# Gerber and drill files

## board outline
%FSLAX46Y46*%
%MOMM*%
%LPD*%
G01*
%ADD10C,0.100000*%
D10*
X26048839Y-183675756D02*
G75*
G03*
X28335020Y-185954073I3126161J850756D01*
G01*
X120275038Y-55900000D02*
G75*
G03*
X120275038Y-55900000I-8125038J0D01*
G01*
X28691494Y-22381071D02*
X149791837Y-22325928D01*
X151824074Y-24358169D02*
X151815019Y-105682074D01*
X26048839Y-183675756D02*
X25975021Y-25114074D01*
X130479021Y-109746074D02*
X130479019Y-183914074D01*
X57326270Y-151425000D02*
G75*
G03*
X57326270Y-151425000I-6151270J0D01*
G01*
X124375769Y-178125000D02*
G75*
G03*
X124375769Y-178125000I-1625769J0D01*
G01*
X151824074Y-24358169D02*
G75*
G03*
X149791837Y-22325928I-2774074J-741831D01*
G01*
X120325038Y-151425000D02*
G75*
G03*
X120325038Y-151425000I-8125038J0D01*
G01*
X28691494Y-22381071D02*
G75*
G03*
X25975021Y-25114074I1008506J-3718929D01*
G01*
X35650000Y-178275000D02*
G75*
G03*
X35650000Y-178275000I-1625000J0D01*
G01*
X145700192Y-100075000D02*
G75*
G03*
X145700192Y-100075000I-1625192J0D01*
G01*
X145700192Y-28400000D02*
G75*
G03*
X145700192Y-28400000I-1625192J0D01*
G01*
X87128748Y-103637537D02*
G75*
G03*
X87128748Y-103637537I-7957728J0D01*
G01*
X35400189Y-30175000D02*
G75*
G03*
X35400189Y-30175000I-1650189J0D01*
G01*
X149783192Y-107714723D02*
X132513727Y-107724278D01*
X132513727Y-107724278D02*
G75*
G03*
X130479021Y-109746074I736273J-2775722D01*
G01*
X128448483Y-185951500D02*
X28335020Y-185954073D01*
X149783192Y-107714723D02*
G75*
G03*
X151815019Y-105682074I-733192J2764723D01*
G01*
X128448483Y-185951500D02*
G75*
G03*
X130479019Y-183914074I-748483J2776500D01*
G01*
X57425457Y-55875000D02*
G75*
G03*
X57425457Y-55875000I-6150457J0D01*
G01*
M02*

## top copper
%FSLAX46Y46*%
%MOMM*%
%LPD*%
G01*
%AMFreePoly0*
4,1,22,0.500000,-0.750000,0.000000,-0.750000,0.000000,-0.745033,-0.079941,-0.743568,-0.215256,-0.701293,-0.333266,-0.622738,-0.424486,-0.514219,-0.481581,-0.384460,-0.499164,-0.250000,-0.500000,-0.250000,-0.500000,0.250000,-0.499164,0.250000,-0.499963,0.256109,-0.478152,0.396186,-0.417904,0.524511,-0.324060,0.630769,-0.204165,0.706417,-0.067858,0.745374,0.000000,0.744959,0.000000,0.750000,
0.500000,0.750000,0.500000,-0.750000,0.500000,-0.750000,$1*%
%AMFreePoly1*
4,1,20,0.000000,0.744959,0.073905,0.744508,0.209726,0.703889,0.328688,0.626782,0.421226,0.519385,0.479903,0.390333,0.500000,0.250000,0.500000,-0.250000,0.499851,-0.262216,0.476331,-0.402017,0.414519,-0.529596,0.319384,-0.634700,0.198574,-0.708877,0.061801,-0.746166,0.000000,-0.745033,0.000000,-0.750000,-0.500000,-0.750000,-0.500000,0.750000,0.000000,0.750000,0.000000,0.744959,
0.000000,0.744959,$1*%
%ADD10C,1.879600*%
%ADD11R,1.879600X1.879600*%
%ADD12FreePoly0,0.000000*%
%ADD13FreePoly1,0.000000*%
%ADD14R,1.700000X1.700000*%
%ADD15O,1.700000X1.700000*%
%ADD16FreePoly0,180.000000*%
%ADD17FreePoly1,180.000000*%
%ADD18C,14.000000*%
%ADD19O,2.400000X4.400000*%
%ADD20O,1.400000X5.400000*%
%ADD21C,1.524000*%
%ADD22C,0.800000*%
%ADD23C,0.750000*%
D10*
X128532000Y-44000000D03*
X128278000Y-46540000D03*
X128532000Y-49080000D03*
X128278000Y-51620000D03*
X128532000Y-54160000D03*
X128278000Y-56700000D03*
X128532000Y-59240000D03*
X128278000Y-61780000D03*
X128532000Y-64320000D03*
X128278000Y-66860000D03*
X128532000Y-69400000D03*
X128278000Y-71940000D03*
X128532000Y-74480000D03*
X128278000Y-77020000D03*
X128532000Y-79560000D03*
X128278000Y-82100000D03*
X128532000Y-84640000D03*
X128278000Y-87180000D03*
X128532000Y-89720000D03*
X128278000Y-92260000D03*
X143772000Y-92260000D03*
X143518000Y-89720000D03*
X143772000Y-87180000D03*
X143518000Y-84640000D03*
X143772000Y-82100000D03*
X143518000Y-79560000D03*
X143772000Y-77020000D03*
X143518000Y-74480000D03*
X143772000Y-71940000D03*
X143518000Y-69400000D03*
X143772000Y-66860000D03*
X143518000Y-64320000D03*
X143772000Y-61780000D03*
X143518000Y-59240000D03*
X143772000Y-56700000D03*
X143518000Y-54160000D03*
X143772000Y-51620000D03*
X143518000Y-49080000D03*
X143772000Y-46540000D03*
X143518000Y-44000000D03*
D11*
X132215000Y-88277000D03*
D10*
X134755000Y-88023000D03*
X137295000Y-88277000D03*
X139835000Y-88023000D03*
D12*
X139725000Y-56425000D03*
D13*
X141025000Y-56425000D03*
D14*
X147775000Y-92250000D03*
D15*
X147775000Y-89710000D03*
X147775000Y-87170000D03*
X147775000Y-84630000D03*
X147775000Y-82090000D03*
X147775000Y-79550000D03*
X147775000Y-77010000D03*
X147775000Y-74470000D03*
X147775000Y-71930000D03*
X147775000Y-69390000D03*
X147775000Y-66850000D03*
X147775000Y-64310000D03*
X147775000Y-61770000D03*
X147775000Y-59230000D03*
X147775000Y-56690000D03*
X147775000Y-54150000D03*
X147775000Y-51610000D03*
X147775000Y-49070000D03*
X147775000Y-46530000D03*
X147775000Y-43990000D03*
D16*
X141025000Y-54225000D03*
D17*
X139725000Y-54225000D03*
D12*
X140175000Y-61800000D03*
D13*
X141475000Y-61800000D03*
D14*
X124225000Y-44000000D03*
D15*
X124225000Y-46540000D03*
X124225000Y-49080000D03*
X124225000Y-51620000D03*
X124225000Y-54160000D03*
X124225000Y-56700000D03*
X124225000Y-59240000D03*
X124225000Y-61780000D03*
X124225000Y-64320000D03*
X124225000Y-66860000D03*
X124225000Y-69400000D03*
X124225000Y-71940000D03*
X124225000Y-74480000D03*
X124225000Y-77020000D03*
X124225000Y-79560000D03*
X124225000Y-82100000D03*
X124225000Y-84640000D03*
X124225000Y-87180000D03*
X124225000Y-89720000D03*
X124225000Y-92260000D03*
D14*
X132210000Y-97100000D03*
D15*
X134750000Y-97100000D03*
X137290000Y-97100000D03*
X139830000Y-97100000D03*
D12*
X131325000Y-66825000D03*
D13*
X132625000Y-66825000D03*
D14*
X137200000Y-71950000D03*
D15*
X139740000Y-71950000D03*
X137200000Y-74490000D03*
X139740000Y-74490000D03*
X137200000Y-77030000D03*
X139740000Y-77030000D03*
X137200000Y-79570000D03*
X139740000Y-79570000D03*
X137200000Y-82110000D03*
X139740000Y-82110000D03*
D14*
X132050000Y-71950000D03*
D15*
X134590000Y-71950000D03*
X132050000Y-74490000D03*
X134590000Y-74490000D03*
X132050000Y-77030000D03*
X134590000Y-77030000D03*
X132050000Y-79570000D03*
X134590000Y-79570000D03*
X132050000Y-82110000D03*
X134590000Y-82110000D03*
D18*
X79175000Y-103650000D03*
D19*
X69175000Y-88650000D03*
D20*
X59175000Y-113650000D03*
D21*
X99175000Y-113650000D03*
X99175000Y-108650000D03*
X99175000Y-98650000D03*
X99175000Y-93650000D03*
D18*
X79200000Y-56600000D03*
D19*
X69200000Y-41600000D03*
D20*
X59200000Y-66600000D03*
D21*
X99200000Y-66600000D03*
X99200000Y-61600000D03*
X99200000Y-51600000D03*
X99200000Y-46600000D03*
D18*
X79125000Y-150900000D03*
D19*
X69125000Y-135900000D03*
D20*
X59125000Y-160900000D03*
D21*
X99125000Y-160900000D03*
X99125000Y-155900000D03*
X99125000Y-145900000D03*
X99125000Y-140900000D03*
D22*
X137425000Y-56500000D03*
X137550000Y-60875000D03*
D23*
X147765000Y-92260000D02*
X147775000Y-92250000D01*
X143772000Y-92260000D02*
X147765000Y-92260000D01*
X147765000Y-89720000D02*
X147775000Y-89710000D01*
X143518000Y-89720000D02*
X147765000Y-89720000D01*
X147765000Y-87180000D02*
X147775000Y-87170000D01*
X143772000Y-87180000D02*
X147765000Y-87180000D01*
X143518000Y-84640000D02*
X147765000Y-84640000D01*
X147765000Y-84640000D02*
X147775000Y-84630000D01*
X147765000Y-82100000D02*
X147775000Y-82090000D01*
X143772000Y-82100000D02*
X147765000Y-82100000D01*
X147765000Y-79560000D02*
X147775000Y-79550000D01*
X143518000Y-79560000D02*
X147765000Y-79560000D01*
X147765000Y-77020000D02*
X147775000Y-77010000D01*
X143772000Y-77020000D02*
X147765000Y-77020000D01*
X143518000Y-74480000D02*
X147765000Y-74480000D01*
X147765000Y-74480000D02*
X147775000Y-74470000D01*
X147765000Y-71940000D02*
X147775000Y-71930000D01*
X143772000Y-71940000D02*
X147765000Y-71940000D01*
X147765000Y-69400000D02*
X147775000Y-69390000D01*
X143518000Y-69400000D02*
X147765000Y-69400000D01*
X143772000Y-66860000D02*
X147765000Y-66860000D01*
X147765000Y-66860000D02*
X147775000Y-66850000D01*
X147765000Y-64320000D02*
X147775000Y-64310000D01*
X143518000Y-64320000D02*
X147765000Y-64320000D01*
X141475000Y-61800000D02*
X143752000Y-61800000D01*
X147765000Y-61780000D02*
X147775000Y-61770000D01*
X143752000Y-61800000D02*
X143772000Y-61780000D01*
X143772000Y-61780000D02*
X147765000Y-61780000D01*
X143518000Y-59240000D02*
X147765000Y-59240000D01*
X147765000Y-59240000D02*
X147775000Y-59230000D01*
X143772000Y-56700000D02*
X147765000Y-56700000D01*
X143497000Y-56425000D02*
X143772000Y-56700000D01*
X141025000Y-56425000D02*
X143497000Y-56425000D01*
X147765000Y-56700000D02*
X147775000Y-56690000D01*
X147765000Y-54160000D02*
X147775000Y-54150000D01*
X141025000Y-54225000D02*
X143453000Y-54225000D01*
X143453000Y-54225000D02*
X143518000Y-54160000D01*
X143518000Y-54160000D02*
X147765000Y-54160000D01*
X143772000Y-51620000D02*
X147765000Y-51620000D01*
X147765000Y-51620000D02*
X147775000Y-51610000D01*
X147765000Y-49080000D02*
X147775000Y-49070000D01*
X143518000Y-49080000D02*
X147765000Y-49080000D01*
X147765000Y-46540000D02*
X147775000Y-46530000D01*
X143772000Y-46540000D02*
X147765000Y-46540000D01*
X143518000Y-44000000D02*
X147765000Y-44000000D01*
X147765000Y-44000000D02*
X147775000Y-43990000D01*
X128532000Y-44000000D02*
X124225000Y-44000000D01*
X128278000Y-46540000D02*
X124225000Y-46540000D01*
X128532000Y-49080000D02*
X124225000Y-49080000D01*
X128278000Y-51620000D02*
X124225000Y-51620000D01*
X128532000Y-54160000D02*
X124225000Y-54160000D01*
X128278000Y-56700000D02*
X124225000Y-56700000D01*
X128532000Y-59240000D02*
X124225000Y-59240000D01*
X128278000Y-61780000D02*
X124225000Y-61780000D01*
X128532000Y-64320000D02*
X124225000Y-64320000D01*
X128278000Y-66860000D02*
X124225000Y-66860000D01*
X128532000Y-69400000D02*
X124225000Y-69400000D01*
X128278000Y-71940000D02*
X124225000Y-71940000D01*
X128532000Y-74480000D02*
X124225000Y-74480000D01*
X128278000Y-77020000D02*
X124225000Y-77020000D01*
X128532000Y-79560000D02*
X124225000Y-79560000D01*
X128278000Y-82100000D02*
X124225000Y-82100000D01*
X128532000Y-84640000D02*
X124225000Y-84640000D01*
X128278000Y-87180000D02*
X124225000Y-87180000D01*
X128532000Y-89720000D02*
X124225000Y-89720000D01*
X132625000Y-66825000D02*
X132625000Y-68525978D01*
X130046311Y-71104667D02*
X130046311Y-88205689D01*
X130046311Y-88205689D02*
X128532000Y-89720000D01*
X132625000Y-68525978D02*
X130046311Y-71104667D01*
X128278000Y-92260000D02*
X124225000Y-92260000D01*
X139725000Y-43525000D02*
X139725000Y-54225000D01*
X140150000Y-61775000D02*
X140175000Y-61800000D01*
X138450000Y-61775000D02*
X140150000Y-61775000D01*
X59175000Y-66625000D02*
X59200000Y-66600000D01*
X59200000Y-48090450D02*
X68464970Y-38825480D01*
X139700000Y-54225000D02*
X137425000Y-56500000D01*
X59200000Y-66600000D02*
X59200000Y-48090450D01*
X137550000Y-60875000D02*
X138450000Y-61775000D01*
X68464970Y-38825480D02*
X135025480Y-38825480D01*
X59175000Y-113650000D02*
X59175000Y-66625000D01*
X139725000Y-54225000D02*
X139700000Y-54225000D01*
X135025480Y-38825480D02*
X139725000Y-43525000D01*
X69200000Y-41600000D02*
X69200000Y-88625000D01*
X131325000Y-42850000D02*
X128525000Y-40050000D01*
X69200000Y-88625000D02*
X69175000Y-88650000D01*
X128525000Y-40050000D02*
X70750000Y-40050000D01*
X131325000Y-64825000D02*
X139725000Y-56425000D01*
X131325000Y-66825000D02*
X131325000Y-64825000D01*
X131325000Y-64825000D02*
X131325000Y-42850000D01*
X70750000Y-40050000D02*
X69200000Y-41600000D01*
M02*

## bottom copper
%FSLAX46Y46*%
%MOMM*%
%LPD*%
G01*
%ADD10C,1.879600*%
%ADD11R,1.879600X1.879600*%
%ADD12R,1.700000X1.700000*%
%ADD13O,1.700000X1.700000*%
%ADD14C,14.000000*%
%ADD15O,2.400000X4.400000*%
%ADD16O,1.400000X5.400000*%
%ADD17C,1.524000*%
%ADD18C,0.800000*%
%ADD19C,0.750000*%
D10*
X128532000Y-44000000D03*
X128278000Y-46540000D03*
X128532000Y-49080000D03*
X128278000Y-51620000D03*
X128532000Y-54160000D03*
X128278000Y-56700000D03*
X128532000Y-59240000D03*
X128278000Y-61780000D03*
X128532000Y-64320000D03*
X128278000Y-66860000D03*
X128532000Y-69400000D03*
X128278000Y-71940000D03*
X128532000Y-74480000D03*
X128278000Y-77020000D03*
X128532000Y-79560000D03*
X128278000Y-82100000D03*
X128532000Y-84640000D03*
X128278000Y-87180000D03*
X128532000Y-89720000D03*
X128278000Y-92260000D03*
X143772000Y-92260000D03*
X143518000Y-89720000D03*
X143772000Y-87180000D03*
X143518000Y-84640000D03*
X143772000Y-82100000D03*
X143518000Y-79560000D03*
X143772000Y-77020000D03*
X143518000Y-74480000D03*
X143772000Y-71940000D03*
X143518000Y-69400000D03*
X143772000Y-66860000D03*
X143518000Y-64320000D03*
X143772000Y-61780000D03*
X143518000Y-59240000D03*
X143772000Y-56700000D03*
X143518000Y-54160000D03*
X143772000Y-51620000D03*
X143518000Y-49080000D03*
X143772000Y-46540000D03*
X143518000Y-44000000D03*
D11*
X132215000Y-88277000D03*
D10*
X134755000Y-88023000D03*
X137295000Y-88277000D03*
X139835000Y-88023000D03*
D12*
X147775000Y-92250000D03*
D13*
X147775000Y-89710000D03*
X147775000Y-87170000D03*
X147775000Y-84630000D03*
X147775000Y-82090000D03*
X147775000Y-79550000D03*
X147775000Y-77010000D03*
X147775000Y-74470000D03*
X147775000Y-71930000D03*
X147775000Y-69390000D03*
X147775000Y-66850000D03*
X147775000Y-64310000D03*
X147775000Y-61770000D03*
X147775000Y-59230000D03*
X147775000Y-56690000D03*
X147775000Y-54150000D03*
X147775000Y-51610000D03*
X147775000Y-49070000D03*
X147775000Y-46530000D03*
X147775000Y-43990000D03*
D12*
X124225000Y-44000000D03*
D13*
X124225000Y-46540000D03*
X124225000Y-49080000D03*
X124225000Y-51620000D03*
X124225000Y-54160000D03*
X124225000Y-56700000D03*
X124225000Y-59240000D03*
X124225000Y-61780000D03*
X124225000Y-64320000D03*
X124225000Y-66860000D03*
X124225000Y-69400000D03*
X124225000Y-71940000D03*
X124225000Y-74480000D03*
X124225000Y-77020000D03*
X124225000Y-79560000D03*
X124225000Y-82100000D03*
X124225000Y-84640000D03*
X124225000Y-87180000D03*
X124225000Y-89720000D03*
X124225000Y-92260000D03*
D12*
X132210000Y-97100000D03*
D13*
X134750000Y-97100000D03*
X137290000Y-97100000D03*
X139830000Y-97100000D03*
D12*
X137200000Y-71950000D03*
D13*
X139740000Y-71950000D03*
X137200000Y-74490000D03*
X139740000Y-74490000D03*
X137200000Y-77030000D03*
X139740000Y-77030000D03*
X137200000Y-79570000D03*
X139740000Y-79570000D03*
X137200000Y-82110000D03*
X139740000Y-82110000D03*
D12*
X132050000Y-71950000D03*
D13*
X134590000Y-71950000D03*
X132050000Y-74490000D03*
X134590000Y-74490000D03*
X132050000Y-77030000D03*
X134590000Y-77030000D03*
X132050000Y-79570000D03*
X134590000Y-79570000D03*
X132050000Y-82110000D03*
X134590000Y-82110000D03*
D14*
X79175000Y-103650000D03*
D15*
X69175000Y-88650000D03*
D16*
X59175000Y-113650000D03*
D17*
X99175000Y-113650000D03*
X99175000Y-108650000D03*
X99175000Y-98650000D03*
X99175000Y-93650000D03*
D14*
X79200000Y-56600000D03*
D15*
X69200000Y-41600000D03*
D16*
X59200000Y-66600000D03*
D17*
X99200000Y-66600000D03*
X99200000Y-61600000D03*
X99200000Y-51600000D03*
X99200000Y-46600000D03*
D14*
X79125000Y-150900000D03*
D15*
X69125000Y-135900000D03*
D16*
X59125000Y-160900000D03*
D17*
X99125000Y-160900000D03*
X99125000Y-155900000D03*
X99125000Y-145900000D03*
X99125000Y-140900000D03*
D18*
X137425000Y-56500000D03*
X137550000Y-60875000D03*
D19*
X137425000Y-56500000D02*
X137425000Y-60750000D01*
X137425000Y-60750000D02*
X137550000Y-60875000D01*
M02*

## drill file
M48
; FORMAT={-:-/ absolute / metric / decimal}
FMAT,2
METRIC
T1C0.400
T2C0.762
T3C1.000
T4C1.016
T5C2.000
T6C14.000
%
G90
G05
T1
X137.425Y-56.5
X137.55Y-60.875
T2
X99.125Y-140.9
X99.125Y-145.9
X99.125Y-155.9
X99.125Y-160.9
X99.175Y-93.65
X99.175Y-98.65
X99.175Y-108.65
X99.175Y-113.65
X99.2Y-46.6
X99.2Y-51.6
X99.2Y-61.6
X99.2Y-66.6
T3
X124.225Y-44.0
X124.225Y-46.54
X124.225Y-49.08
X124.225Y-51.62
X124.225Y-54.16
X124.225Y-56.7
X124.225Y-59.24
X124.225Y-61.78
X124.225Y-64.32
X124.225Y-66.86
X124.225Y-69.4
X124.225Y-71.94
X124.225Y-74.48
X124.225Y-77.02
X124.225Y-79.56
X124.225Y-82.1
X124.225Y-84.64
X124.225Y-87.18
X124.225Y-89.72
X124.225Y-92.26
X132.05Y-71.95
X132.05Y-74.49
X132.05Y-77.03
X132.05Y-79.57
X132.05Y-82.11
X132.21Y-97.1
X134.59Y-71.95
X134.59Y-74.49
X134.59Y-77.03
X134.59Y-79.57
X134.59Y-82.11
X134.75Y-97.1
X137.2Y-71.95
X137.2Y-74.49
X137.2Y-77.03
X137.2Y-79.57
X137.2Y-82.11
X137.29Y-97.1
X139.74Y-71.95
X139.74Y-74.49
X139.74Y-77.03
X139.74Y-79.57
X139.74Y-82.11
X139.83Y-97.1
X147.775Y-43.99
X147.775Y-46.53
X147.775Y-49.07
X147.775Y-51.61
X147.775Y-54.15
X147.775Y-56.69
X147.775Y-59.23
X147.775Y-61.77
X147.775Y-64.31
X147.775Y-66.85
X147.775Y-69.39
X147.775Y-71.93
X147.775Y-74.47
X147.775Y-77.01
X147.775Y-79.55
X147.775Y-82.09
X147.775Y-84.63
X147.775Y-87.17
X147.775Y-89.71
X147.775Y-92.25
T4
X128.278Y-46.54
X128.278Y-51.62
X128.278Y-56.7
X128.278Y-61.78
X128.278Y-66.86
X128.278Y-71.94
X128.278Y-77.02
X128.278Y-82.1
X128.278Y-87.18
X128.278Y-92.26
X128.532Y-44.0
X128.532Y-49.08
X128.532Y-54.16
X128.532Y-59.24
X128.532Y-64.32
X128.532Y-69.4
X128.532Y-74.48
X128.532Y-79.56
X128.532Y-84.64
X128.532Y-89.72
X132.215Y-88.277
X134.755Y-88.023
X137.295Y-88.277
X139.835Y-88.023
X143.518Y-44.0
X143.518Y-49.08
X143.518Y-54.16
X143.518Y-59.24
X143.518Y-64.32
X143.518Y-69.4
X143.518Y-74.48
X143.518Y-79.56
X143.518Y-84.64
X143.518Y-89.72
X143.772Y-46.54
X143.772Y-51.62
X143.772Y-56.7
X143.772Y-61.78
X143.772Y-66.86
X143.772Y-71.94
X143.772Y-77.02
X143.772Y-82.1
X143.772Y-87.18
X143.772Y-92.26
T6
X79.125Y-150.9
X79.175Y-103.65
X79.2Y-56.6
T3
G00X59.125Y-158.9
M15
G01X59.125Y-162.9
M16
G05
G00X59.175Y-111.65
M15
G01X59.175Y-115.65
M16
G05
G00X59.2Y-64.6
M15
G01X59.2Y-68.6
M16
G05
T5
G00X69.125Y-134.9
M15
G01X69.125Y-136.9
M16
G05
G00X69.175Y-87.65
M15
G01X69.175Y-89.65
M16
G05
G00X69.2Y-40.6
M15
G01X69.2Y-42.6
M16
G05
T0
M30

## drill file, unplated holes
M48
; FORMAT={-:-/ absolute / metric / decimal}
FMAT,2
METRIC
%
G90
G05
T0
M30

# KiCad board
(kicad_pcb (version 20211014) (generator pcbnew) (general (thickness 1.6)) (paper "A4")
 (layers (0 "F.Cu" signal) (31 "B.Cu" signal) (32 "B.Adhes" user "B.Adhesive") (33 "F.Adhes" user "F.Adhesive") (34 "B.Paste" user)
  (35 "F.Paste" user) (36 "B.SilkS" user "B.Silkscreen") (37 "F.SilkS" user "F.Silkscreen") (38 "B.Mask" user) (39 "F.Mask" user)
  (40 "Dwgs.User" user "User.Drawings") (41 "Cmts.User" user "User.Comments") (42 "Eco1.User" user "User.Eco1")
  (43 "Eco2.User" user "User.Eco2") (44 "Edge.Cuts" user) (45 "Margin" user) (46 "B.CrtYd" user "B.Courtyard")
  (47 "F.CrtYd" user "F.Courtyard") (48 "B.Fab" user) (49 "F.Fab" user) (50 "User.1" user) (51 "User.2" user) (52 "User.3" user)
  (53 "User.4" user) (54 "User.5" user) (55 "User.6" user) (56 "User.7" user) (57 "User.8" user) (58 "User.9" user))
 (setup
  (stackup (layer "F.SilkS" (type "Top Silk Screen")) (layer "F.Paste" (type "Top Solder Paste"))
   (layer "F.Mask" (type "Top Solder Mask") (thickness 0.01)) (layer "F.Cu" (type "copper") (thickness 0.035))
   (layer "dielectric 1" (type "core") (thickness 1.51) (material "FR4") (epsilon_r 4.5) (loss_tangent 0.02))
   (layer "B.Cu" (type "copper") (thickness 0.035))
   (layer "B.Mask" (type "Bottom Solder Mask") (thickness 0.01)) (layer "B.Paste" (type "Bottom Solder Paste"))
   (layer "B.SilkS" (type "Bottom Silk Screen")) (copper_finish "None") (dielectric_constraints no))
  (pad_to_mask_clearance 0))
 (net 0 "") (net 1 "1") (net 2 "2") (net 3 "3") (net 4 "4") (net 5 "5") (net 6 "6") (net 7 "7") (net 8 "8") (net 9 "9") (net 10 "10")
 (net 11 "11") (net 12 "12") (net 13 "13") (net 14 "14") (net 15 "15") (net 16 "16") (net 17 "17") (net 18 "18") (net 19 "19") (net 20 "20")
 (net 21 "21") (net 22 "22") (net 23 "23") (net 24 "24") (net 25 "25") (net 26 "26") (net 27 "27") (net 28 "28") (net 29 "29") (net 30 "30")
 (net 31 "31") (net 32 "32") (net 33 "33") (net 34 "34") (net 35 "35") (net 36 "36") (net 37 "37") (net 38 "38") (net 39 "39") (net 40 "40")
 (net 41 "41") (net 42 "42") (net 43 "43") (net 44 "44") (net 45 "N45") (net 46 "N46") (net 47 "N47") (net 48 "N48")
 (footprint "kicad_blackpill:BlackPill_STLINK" (layer "F.Cu") (at 136.025 69.1)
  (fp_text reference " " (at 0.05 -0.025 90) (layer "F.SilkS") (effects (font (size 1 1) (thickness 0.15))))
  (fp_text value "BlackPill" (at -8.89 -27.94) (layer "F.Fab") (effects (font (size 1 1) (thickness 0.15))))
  (pad "1" thru_hole circle (at -7.493 -25.1 270) (size 1.8796 1.8796) (drill 1.016) (layers *.Cu *.Mask) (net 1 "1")
   (solder_mask_margin 0.1016))
  (pad "2" thru_hole circle (at -7.747 -22.56 270) (size 1.8796 1.8796) (drill 1.016) (layers *.Cu *.Mask) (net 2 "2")
   (solder_mask_margin 0.1016))
  (pad "3" thru_hole circle (at -7.493 -20.02 270) (size 1.8796 1.8796) (drill 1.016) (layers *.Cu *.Mask) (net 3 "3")
   (solder_mask_margin 0.1016))
  (pad "4" thru_hole circle (at -7.747 -17.48 270) (size 1.8796 1.8796) (drill 1.016) (layers *.Cu *.Mask) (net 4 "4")
   (solder_mask_margin 0.1016))
  (pad "5" thru_hole circle (at -7.493 -14.94 270) (size 1.8796 1.8796) (drill 1.016) (layers *.Cu *.Mask) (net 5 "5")
   (solder_mask_margin 0.1016))
  (pad "6" thru_hole circle (at -7.747 -12.4 270) (size 1.8796 1.8796) (drill 1.016) (layers *.Cu *.Mask) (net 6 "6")
   (solder_mask_margin 0.1016))
  (pad "7" thru_hole circle (at -7.493 -9.86 270) (size 1.8796 1.8796) (drill 1.016) (layers *.Cu *.Mask) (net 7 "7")
   (solder_mask_margin 0.1016))
  (pad "8" thru_hole circle (at -7.747 -7.32 270) (size 1.8796 1.8796) (drill 1.016) (layers *.Cu *.Mask) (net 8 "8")
   (solder_mask_margin 0.1016))
  (pad "9" thru_hole circle (at -7.493 -4.78 270) (size 1.8796 1.8796) (drill 1.016) (layers *.Cu *.Mask) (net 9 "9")
   (solder_mask_margin 0.1016))
  (pad "10" thru_hole circle (at -7.747 -2.24 270) (size 1.8796 1.8796) (drill 1.016) (layers *.Cu *.Mask) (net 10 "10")
   (solder_mask_margin 0.1016))
  (pad "11" thru_hole circle (at -7.493 0.3 270) (size 1.8796 1.8796) (drill 1.016) (layers *.Cu *.Mask) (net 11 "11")
   (solder_mask_margin 0.1016))
  (pad "12" thru_hole circle (at -7.747 2.84 270) (size 1.8796 1.8796) (drill 1.016) (layers *.Cu *.Mask) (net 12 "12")
   (solder_mask_margin 0.1016))
  (pad "13" thru_hole circle (at -7.493 5.38 270) (size 1.8796 1.8796) (drill 1.016) (layers *.Cu *.Mask) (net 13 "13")
   (solder_mask_margin 0.1016))
  (pad "14" thru_hole circle (at -7.747 7.92 270) (size 1.8796 1.8796) (drill 1.016) (layers *.Cu *.Mask) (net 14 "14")
   (solder_mask_margin 0.1016))
  (pad "15" thru_hole circle (at -7.493 10.46 270) (size 1.8796 1.8796) (drill 1.016) (layers *.Cu *.Mask) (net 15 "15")
   (solder_mask_margin 0.1016))
  (pad "16" thru_hole circle (at -7.747 13 270) (size 1.8796 1.8796) (drill 1.016) (layers *.Cu *.Mask) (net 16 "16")
   (solder_mask_margin 0.1016))
  (pad "17" thru_hole circle (at -7.493 15.54 270) (size 1.8796 1.8796) (drill 1.016) (layers *.Cu *.Mask) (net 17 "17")
   (solder_mask_margin 0.1016))
  (pad "18" thru_hole circle (at -7.747 18.08 270) (size 1.8796 1.8796) (drill 1.016) (layers *.Cu *.Mask) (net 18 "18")
   (solder_mask_margin 0.1016))
  (pad "19" thru_hole circle (at -7.493 20.62 270) (size 1.8796 1.8796) (drill 1.016) (layers *.Cu *.Mask) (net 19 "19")
   (solder_mask_margin 0.1016))
  (pad "20" thru_hole circle (at -7.747 23.16 270) (size 1.8796 1.8796) (drill 1.016) (layers *.Cu *.Mask) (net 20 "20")
   (solder_mask_margin 0.1016))
  (pad "21" thru_hole circle (at 7.747 23.16 90) (size 1.8796 1.8796) (drill 1.016) (layers *.Cu *.Mask) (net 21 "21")
   (solder_mask_margin 0.1016))
  (pad "22" thru_hole circle (at 7.493 20.62 90) (size 1.8796 1.8796) (drill 1.016) (layers *.Cu *.Mask) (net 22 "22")
   (solder_mask_margin 0.1016))
  (pad "23" thru_hole circle (at 7.747 18.08 90) (size 1.8796 1.8796) (drill 1.016) (layers *.Cu *.Mask) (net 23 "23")
   (solder_mask_margin 0.1016))
  (pad "24" thru_hole circle (at 7.493 15.54 90) (size 1.8796 1.8796) (drill 1.016) (layers *.Cu *.Mask) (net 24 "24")
   (solder_mask_margin 0.1016))
  (pad "25" thru_hole circle (at 7.747 13 90) (size 1.8796 1.8796) (drill 1.016) (layers *.Cu *.Mask) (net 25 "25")
   (solder_mask_margin 0.1016))
  (pad "26" thru_hole circle (at 7.493 10.46 90) (size 1.8796 1.8796) (drill 1.016) (layers *.Cu *.Mask) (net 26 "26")
   (solder_mask_margin 0.1016))
  (pad "27" thru_hole circle (at 7.747 7.92 90) (size 1.8796 1.8796) (drill 1.016) (layers *.Cu *.Mask) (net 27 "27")
   (solder_mask_margin 0.1016))
  (pad "28" thru_hole circle (at 7.493 5.38 90) (size 1.8796 1.8796) (drill 1.016) (layers *.Cu *.Mask) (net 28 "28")
   (solder_mask_margin 0.1016))
  (pad "29" thru_hole circle (at 7.747 2.84 90) (size 1.8796 1.8796) (drill 1.016) (layers *.Cu *.Mask) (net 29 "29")
   (solder_mask_margin 0.1016))
  (pad "30" thru_hole circle (at 7.493 0.3 90) (size 1.8796 1.8796) (drill 1.016) (layers *.Cu *.Mask) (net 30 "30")
   (solder_mask_margin 0.1016))
  (pad "31" thru_hole circle (at 7.747 -2.24 90) (size 1.8796 1.8796) (drill 1.016) (layers *.Cu *.Mask) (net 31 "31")
   (solder_mask_margin 0.1016))
  (pad "32" thru_hole circle (at 7.493 -4.78 90) (size 1.8796 1.8796) (drill 1.016) (layers *.Cu *.Mask) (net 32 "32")
   (solder_mask_margin 0.1016))
  (pad "33" thru_hole circle (at 7.747 -7.32 90) (size 1.8796 1.8796) (drill 1.016) (layers *.Cu *.Mask) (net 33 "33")
   (solder_mask_margin 0.1016))
  (pad "34" thru_hole circle (at 7.493 -9.86 90) (size 1.8796 1.8796) (drill 1.016) (layers *.Cu *.Mask) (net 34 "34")
   (solder_mask_margin 0.1016))
  (pad "35" thru_hole circle (at 7.747 -12.4 90) (size 1.8796 1.8796) (drill 1.016) (layers *.Cu *.Mask) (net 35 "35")
   (solder_mask_margin 0.1016))
  (pad "36" thru_hole circle (at 7.493 -14.94 90) (size 1.8796 1.8796) (drill 1.016) (layers *.Cu *.Mask) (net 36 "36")
   (solder_mask_margin 0.1016))
  (pad "37" thru_hole circle (at 7.747 -17.48 90) (size 1.8796 1.8796) (drill 1.016) (layers *.Cu *.Mask) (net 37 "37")
   (solder_mask_margin 0.1016))
  (pad "38" thru_hole circle (at 7.493 -20.02 90) (size 1.8796 1.8796) (drill 1.016) (layers *.Cu *.Mask) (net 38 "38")
   (solder_mask_margin 0.1016))
  (pad "39" thru_hole circle (at 7.747 -22.56 90) (size 1.8796 1.8796) (drill 1.016) (layers *.Cu *.Mask) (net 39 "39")
   (solder_mask_margin 0.1016))
  (pad "40" thru_hole circle (at 7.493 -25.1 90) (size 1.8796 1.8796) (drill 1.016) (layers *.Cu *.Mask) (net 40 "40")
   (solder_mask_margin 0.1016))
  (pad "41" thru_hole rect (at -3.81 19.177 90) (size 1.8796 1.8796) (drill 1.016) (layers *.Cu *.Mask) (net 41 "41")
   (solder_mask_margin 0.1016))
  (pad "42" thru_hole circle (at -1.27 18.923 90) (size 1.8796 1.8796) (drill 1.016) (layers *.Cu *.Mask) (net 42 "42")
   (solder_mask_margin 0.1016))
  (pad "43" thru_hole circle (at 1.27 19.177 90) (size 1.8796 1.8796) (drill 1.016) (layers *.Cu *.Mask) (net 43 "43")
   (solder_mask_margin 0.1016))
  (pad "44" thru_hole circle (at 3.81 18.923 90) (size 1.8796 1.8796) (drill 1.016) (layers *.Cu *.Mask) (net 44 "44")
   (solder_mask_margin 0.1016)))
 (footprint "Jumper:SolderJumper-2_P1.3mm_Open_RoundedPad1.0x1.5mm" (layer "F.Cu") (at 140.375 56.425)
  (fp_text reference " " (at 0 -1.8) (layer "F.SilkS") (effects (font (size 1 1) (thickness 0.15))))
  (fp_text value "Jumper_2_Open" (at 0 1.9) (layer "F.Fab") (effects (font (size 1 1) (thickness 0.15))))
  (pad "1" smd custom (at -0.65 0) (size 1 0.5) (layers "F.Cu" "F.Mask") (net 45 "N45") (zone_connect 2)
   (options (clearance outline) (anchor rect)) (primitives))
  (pad "2" smd custom (at 0.65 0) (size 1 0.5) (layers "F.Cu" "F.Mask") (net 35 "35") (zone_connect 2)
   (options (clearance outline) (anchor rect)) (primitives)))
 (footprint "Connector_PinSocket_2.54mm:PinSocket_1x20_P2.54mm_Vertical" (layer "F.Cu") (at 147.775 92.25 180)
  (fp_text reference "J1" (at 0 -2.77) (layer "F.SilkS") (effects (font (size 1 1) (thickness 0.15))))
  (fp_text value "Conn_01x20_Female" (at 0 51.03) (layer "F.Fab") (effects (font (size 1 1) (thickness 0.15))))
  (pad "1" thru_hole rect (at 0 0 180) (size 1.7 1.7) (drill 1) (layers *.Cu *.Mask) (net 21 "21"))
  (pad "2" thru_hole oval (at 0 2.54 180) (size 1.7 1.7) (drill 1) (layers *.Cu *.Mask) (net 22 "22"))
  (pad "3" thru_hole oval (at 0 5.08 180) (size 1.7 1.7) (drill 1) (layers *.Cu *.Mask) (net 23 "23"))
  (pad "4" thru_hole oval (at 0 7.62 180) (size 1.7 1.7) (drill 1) (layers *.Cu *.Mask) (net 24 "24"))
  (pad "5" thru_hole oval (at 0 10.16 180) (size 1.7 1.7) (drill 1) (layers *.Cu *.Mask) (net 25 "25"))
  (pad "6" thru_hole oval (at 0 12.7 180) (size 1.7 1.7) (drill 1) (layers *.Cu *.Mask) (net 26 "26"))
  (pad "7" thru_hole oval (at 0 15.24 180) (size 1.7 1.7) (drill 1) (layers *.Cu *.Mask) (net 27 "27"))
  (pad "8" thru_hole oval (at 0 17.78 180) (size 1.7 1.7) (drill 1) (layers *.Cu *.Mask) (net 28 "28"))
  (pad "9" thru_hole oval (at 0 20.32 180) (size 1.7 1.7) (drill 1) (layers *.Cu *.Mask) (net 29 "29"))
  (pad "10" thru_hole oval (at 0 22.86 180) (size 1.7 1.7) (drill 1) (layers *.Cu *.Mask) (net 30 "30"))
  (pad "11" thru_hole oval (at 0 25.4 180) (size 1.7 1.7) (drill 1) (layers *.Cu *.Mask) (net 31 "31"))
  (pad "12" thru_hole oval (at 0 27.94 180) (size 1.7 1.7) (drill 1) (layers *.Cu *.Mask) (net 32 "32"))
  (pad "13" thru_hole oval (at 0 30.48 180) (size 1.7 1.7) (drill 1) (layers *.Cu *.Mask) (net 33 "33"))
  (pad "14" thru_hole oval (at 0 33.02 180) (size 1.7 1.7) (drill 1) (layers *.Cu *.Mask) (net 34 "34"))
  (pad "15" thru_hole oval (at 0 35.56 180) (size 1.7 1.7) (drill 1) (layers *.Cu *.Mask) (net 35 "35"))
  (pad "16" thru_hole oval (at 0 38.1 180) (size 1.7 1.7) (drill 1) (layers *.Cu *.Mask) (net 36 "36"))
  (pad "17" thru_hole oval (at 0 40.64 180) (size 1.7 1.7) (drill 1) (layers *.Cu *.Mask) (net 37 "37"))
  (pad "18" thru_hole oval (at 0 43.18 180) (size 1.7 1.7) (drill 1) (layers *.Cu *.Mask) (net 38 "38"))
  (pad "19" thru_hole oval (at 0 45.72 180) (size 1.7 1.7) (drill 1) (layers *.Cu *.Mask) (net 39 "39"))
  (pad "20" thru_hole oval (at 0 48.26 180) (size 1.7 1.7) (drill 1) (layers *.Cu *.Mask) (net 40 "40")))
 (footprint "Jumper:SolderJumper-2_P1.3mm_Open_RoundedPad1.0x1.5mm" (layer "F.Cu") (at 140.375 54.225 180)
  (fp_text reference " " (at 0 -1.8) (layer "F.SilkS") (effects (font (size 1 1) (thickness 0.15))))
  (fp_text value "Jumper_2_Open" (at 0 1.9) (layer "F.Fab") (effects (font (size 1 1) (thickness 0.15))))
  (pad "1" smd custom (at -0.65 0 180) (size 1 0.5) (layers "F.Cu" "F.Mask") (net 36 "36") (zone_connect 2)
   (options (clearance outline) (anchor rect)) (primitives))
  (pad "2" smd custom (at 0.65 0 180) (size 1 0.5) (layers "F.Cu" "F.Mask") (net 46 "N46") (zone_connect 2)
   (options (clearance outline) (anchor rect)) (primitives)))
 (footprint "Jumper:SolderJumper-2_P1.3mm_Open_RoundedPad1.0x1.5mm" (layer "F.Cu") (at 140.825 61.8)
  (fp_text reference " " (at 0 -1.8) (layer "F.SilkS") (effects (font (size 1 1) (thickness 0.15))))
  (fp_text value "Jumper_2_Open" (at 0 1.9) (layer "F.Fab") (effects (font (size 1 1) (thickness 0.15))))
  (pad "1" smd custom (at -0.65 0) (size 1 0.5) (layers "F.Cu" "F.Mask") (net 46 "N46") (zone_connect 2)
   (options (clearance outline) (anchor rect)) (primitives))
  (pad "2" smd custom (at 0.65 0) (size 1 0.5) (layers "F.Cu" "F.Mask") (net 33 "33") (zone_connect 2)
   (options (clearance outline) (anchor rect)) (primitives)))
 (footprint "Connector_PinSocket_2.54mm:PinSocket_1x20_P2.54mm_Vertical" (layer "F.Cu") (at 124.225 44)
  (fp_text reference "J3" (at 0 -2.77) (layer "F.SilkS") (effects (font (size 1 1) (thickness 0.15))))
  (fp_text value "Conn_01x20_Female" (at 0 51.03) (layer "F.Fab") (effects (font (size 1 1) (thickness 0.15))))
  (pad "1" thru_hole rect (at 0 0) (size 1.7 1.7) (drill 1) (layers *.Cu *.Mask) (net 1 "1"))
  (pad "2" thru_hole oval (at 0 2.54) (size 1.7 1.7) (drill 1) (layers *.Cu *.Mask) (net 2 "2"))
  (pad "3" thru_hole oval (at 0 5.08) (size 1.7 1.7) (drill 1) (layers *.Cu *.Mask) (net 3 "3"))
  (pad "4" thru_hole oval (at 0 7.62) (size 1.7 1.7) (drill 1) (layers *.Cu *.Mask) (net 4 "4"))
  (pad "5" thru_hole oval (at 0 10.16) (size 1.7 1.7) (drill 1) (layers *.Cu *.Mask) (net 5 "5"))
  (pad "6" thru_hole oval (at 0 12.7) (size 1.7 1.7) (drill 1) (layers *.Cu *.Mask) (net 6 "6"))
  (pad "7" thru_hole oval (at 0 15.24) (size 1.7 1.7) (drill 1) (layers *.Cu *.Mask) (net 7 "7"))
  (pad "8" thru_hole oval (at 0 17.78) (size 1.7 1.7) (drill 1) (layers *.Cu *.Mask) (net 8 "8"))
  (pad "9" thru_hole oval (at 0 20.32) (size 1.7 1.7) (drill 1) (layers *.Cu *.Mask) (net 9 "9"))
  (pad "10" thru_hole oval (at 0 22.86) (size 1.7 1.7) (drill 1) (layers *.Cu *.Mask) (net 10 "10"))
  (pad "11" thru_hole oval (at 0 25.4) (size 1.7 1.7) (drill 1) (layers *.Cu *.Mask) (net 11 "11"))
  (pad "12" thru_hole oval (at 0 27.94) (size 1.7 1.7) (drill 1) (layers *.Cu *.Mask) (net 12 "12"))
  (pad "13" thru_hole oval (at 0 30.48) (size 1.7 1.7) (drill 1) (layers *.Cu *.Mask) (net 13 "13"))
  (pad "14" thru_hole oval (at 0 33.02) (size 1.7 1.7) (drill 1) (layers *.Cu *.Mask) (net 14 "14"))
  (pad "15" thru_hole oval (at 0 35.56) (size 1.7 1.7) (drill 1) (layers *.Cu *.Mask) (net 15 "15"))
  (pad "16" thru_hole oval (at 0 38.1) (size 1.7 1.7) (drill 1) (layers *.Cu *.Mask) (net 16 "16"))
  (pad "17" thru_hole oval (at 0 40.64) (size 1.7 1.7) (drill 1) (layers *.Cu *.Mask) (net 17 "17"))
  (pad "18" thru_hole oval (at 0 43.18) (size 1.7 1.7) (drill 1) (layers *.Cu *.Mask) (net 18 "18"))
  (pad "19" thru_hole oval (at 0 45.72) (size 1.7 1.7) (drill 1) (layers *.Cu *.Mask) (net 19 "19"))
  (pad "20" thru_hole oval (at 0 48.26) (size 1.7 1.7) (drill 1) (layers *.Cu *.Mask) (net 20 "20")))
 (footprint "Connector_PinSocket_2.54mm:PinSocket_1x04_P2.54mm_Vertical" (layer "F.Cu") (at 132.21 97.1 90)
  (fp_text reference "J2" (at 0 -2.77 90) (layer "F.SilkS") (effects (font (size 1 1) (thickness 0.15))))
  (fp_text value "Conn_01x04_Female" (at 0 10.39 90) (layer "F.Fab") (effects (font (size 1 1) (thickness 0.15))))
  (pad "1" thru_hole rect (at 0 0 90) (size 1.7 1.7) (drill 1) (layers *.Cu *.Mask) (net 41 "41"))
  (pad "2" thru_hole oval (at 0 2.54 90) (size 1.7 1.7) (drill 1) (layers *.Cu *.Mask) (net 42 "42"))
  (pad "3" thru_hole oval (at 0 5.08 90) (size 1.7 1.7) (drill 1) (layers *.Cu *.Mask) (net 43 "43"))
  (pad "4" thru_hole oval (at 0 7.62 90) (size 1.7 1.7) (drill 1) (layers *.Cu *.Mask) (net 44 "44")))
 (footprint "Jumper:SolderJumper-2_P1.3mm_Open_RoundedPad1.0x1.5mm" (layer "F.Cu") (at 131.975 66.825)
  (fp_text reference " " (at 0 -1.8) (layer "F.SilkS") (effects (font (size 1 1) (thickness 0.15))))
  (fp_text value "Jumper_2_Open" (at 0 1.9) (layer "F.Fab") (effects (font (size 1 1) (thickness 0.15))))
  (pad "1" smd custom (at -0.65 0) (size 1 0.5) (layers "F.Cu" "F.Mask") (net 45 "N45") (zone_connect 2)
   (options (clearance outline) (anchor rect)) (primitives))
  (pad "2" smd custom (at 0.65 0) (size 1 0.5) (layers "F.Cu" "F.Mask") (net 19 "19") (zone_connect 2)
   (options (clearance outline) (anchor rect)) (primitives)))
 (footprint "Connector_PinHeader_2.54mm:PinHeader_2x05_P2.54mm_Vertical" (layer "F.Cu") (at 137.2 71.95)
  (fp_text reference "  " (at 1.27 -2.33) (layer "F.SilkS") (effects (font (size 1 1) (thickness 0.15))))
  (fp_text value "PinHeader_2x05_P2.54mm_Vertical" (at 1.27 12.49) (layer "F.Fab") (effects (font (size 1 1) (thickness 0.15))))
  (pad "1" thru_hole rect (at 0 0) (size 1.7 1.7) (drill 1) (layers *.Cu *.Mask))
  (pad "2" thru_hole oval (at 2.54 0) (size 1.7 1.7) (drill 1) (layers *.Cu *.Mask))
  (pad "3" thru_hole oval (at 0 2.54) (size 1.7 1.7) (drill 1) (layers *.Cu *.Mask))
  (pad "4" thru_hole oval (at 2.54 2.54) (size 1.7 1.7) (drill 1) (layers *.Cu *.Mask))
  (pad "5" thru_hole oval (at 0 5.08) (size 1.7 1.7) (drill 1) (layers *.Cu *.Mask))
  (pad "6" thru_hole oval (at 2.54 5.08) (size 1.7 1.7) (drill 1) (layers *.Cu *.Mask))
  (pad "7" thru_hole oval (at 0 7.62) (size 1.7 1.7) (drill 1) (layers *.Cu *.Mask))
  (pad "8" thru_hole oval (at 2.54 7.62) (size 1.7 1.7) (drill 1) (layers *.Cu *.Mask))
  (pad "9" thru_hole oval (at 0 10.16) (size 1.7 1.7) (drill 1) (layers *.Cu *.Mask))
  (pad "10" thru_hole oval (at 2.54 10.16) (size 1.7 1.7) (drill 1) (layers *.Cu *.Mask)))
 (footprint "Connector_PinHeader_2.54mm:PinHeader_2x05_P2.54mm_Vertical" (layer "F.Cu") (at 132.05 71.95)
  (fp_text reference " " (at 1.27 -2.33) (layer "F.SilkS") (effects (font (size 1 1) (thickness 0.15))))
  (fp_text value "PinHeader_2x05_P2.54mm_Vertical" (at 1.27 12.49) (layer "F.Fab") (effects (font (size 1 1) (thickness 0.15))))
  (pad "1" thru_hole rect (at 0 0) (size 1.7 1.7) (drill 1) (layers *.Cu *.Mask))
  (pad "2" thru_hole oval (at 2.54 0) (size 1.7 1.7) (drill 1) (layers *.Cu *.Mask))
  (pad "3" thru_hole oval (at 0 2.54) (size 1.7 1.7) (drill 1) (layers *.Cu *.Mask))
  (pad "4" thru_hole oval (at 2.54 2.54) (size 1.7 1.7) (drill 1) (layers *.Cu *.Mask))
  (pad "5" thru_hole oval (at 0 5.08) (size 1.7 1.7) (drill 1) (layers *.Cu *.Mask))
  (pad "6" thru_hole oval (at 2.54 5.08) (size 1.7 1.7) (drill 1) (layers *.Cu *.Mask))
  (pad "7" thru_hole oval (at 0 7.62) (size 1.7 1.7) (drill 1) (layers *.Cu *.Mask))
  (pad "8" thru_hole oval (at 2.54 7.62) (size 1.7 1.7) (drill 1) (layers *.Cu *.Mask))
  (pad "9" thru_hole oval (at 0 10.16) (size 1.7 1.7) (drill 1) (layers *.Cu *.Mask))
  (pad "10" thru_hole oval (at 2.54 10.16) (size 1.7 1.7) (drill 1) (layers *.Cu *.Mask)))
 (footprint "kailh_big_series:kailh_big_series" (layer "B.Cu") (at 79.175 103.65 -90)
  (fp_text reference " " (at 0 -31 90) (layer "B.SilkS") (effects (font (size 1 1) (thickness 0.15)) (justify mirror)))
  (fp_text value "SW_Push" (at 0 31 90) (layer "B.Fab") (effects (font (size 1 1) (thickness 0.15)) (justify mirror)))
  (pad "" thru_hole circle (at 0 0 270) (size 14 14) (drill 14) (layers *.Cu *.Mask))
  (pad "1" thru_hole oval (at -15 10 270) (size 4.4 2.4) (drill oval 4 2) (layers *.Cu *.Mask) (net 45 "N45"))
  (pad "2" thru_hole oval (at 10 20 270) (size 5.4 1.4) (drill oval 5 1) (layers *.Cu *.Mask) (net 46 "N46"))
  (pad "4" thru_hole circle (at 10 -20 270) (size 1.524 1.524) (drill 0.762) (layers *.Cu *.Mask))
  (pad "5" thru_hole circle (at 5 -20 270) (size 1.524 1.524) (drill 0.762) (layers *.Cu *.Mask))
  (pad "6" thru_hole circle (at -5 -20 270) (size 1.524 1.524) (drill 0.762) (layers *.Cu *.Mask))
  (pad "7" thru_hole circle (at -10 -20 270) (size 1.524 1.524) (drill 0.762) (layers *.Cu *.Mask)))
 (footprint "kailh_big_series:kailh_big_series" (layer "B.Cu") (at 79.2 56.6 -90)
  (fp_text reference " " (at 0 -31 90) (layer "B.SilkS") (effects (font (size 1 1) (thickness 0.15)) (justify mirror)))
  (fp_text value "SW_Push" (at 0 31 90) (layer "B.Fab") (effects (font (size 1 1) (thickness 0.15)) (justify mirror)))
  (pad "" thru_hole circle (at 0 0 270) (size 14 14) (drill 14) (layers *.Cu *.Mask))
  (pad "1" thru_hole oval (at -15 10 270) (size 4.4 2.4) (drill oval 4 2) (layers *.Cu *.Mask) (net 45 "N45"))
  (pad "2" thru_hole oval (at 10 20 270) (size 5.4 1.4) (drill oval 5 1) (layers *.Cu *.Mask) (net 46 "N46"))
  (pad "4" thru_hole circle (at 10 -20 270) (size 1.524 1.524) (drill 0.762) (layers *.Cu *.Mask))
  (pad "5" thru_hole circle (at 5 -20 270) (size 1.524 1.524) (drill 0.762) (layers *.Cu *.Mask))
  (pad "6" thru_hole circle (at -5 -20 270) (size 1.524 1.524) (drill 0.762) (layers *.Cu *.Mask))
  (pad "7" thru_hole circle (at -10 -20 270) (size 1.524 1.524) (drill 0.762) (layers *.Cu *.Mask)))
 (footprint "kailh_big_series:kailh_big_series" (layer "B.Cu") (at 79.125 150.9 -90)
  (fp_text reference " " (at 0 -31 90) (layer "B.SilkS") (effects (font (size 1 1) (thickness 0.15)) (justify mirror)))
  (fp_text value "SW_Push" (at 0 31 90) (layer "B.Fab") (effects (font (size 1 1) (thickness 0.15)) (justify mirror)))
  (pad "" thru_hole circle (at 0 0 270) (size 14 14) (drill 14) (layers *.Cu *.Mask))
  (pad "1" thru_hole oval (at -15 10 270) (size 4.4 2.4) (drill oval 4 2) (layers *.Cu *.Mask) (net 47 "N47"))
  (pad "2" thru_hole oval (at 10 20 270) (size 5.4 1.4) (drill oval 5 1) (layers *.Cu *.Mask) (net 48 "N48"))
  (pad "4" thru_hole circle (at 10 -20 270) (size 1.524 1.524) (drill 0.762) (layers *.Cu *.Mask))
  (pad "5" thru_hole circle (at 5 -20 270) (size 1.524 1.524) (drill 0.762) (layers *.Cu *.Mask))
  (pad "6" thru_hole circle (at -5 -20 270) (size 1.524 1.524) (drill 0.762) (layers *.Cu *.Mask))
  (pad "7" thru_hole circle (at -10 -20 270) (size 1.524 1.524) (drill 0.762) (layers *.Cu *.Mask)))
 (gr_arc (start 28.33502 185.954073) (mid 26.888026 185.119867) (end 26.048839 183.675756) (layer "Edge.Cuts") (width 0.1))
 (gr_circle (center 112.15 55.9) (end 120.275 55.875) (layer "Edge.Cuts") (width 0.1) (fill none))
 (gr_line (start 28.691494 22.381071) (end 149.791837 22.325928) (layer "Edge.Cuts") (width 0.1))
 (gr_line (start 151.824074 24.358169) (end 151.815019 105.682074) (layer "Edge.Cuts") (width 0.1))
 (gr_line (start 26.048839 183.675756) (end 25.975021 25.114074) (layer "Edge.Cuts") (width 0.1))
 (gr_line (start 130.479021 109.746074) (end 130.479019 183.914074) (layer "Edge.Cuts") (width 0.1))
 (gr_circle (center 51.175 151.425) (end 57.325 151.55) (layer "Edge.Cuts") (width 0.1) (fill none))
 (gr_circle (center 122.75 178.125) (end 124.375 178.075) (layer "Edge.Cuts") (width 0.1) (fill none))
 (gr_arc (start 149.791837 22.325928) (mid 151.080494 23.06951) (end 151.824074 24.358169) (layer "Edge.Cuts") (width 0.1))
 (gr_circle (center 112.2 151.425) (end 120.325 151.4) (layer "Edge.Cuts") (width 0.1) (fill none))
 (gr_arc (start 25.975021 25.114074) (mid 26.96709 23.38362) (end 28.691494 22.381071) (layer "Edge.Cuts") (width 0.1))
 (gr_circle (center 34.025 178.275) (end 35.65 178.275) (layer "Edge.Cuts") (width 0.1) (fill none))
 (gr_circle (center 144.075 100.075) (end 145.7 100.05) (layer "Edge.Cuts") (width 0.1) (fill none))
 (gr_circle (center 144.075 28.4) (end 145.7 28.425) (layer "Edge.Cuts") (width 0.1) (fill none))
 (gr_circle (center 79.17102 103.637537) (end 84.175 97.45) (layer "Edge.Cuts") (width 0.1) (fill none))
 (gr_circle (center 33.75 30.175) (end 35.4 30.15) (layer "Edge.Cuts") (width 0.1) (fill none))
 (gr_line (start 149.783192 107.714723) (end 132.513727 107.724278) (layer "Edge.Cuts") (width 0.1))
 (gr_arc (start 130.479021 109.746074) (mid 131.225866 108.462941) (end 132.513727 107.724278) (layer "Edge.Cuts") (width 0.1))
 (gr_line (start 128.448483 185.9515) (end 28.33502 185.954073) (layer "Edge.Cuts") (width 0.1))
 (gr_arc (start 151.815019 105.682074) (mid 151.07294 106.972122) (end 149.783192 107.714723) (layer "Edge.Cuts") (width 0.1))
 (gr_arc (start 130.479019 183.914074) (mid 129.73681 185.204922) (end 128.448483 185.9515) (layer "Edge.Cuts") (width 0.1))
 (gr_circle (center 51.275 55.875) (end 57.425 55.8) (layer "Edge.Cuts") (width 0.1) (fill none))
 (segment (start 147.765 92.26) (end 147.775 92.25) (width 0.75) (layer "F.Cu") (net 21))
 (segment (start 143.772 92.26) (end 147.765 92.26) (width 0.75) (layer "F.Cu") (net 21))
 (segment (start 147.765 89.72) (end 147.775 89.71) (width 0.75) (layer "F.Cu") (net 22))
 (segment (start 143.518 89.72) (end 147.765 89.72) (width 0.75) (layer "F.Cu") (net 22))
 (segment (start 147.765 87.18) (end 147.775 87.17) (width 0.75) (layer "F.Cu") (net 23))
 (segment (start 143.772 87.18) (end 147.765 87.18) (width 0.75) (layer "F.Cu") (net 23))
 (segment (start 143.518 84.64) (end 147.765 84.64) (width 0.75) (layer "F.Cu") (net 24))
 (segment (start 147.765 84.64) (end 147.775 84.63) (width 0.75) (layer "F.Cu") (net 24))
 (segment (start 147.765 82.1) (end 147.775 82.09) (width 0.75) (layer "F.Cu") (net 25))
 (segment (start 143.772 82.1) (end 147.765 82.1) (width 0.75) (layer "F.Cu") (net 25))
 (segment (start 147.765 79.56) (end 147.775 79.55) (width 0.75) (layer "F.Cu") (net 26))
 (segment (start 143.518 79.56) (end 147.765 79.56) (width 0.75) (layer "F.Cu") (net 26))
 (segment (start 147.765 77.02) (end 147.775 77.01) (width 0.75) (layer "F.Cu") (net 27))
 (segment (start 143.772 77.02) (end 147.765 77.02) (width 0.75) (layer "F.Cu") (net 27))
 (segment (start 143.518 74.48) (end 147.765 74.48) (width 0.75) (layer "F.Cu") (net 28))
 (segment (start 147.765 74.48) (end 147.775 74.47) (width 0.75) (layer "F.Cu") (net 28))
 (segment (start 147.765 71.94) (end 147.775 71.93) (width 0.75) (layer "F.Cu") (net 29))
 (segment (start 143.772 71.94) (end 147.765 71.94) (width 0.75) (layer "F.Cu") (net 29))
 (segment (start 147.765 69.4) (end 147.775 69.39) (width 0.75) (layer "F.Cu") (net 30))
 (segment (start 143.518 69.4) (end 147.765 69.4) (width 0.75) (layer "F.Cu") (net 30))
 (segment (start 143.772 66.86) (end 147.765 66.86) (width 0.75) (layer "F.Cu") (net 31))
 (segment (start 147.765 66.86) (end 147.775 66.85) (width 0.75) (layer "F.Cu") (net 31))
 (segment (start 147.765 64.32) (end 147.775 64.31) (width 0.75) (layer "F.Cu") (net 32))
 (segment (start 143.518 64.32) (end 147.765 64.32) (width 0.75) (layer "F.Cu") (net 32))
 (segment (start 141.475 61.8) (end 143.752 61.8) (width 0.75) (layer "F.Cu") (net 33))
 (segment (start 147.765 61.78) (end 147.775 61.77) (width 0.75) (layer "F.Cu") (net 33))
 (segment (start 143.752 61.8) (end 143.772 61.78) (width 0.75) (layer "F.Cu") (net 33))
 (segment (start 143.772 61.78) (end 147.765 61.78) (width 0.75) (layer "F.Cu") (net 33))
 (segment (start 143.518 59.24) (end 147.765 59.24) (width 0.75) (layer "F.Cu") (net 34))
 (segment (start 147.765 59.24) (end 147.775 59.23) (width 0.75) (layer "F.Cu") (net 34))
 (segment (start 143.772 56.7) (end 147.765 56.7) (width 0.75) (layer "F.Cu") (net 35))
 (segment (start 143.497 56.425) (end 143.772 56.7) (width 0.75) (layer "F.Cu") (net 35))
 (segment (start 141.025 56.425) (end 143.497 56.425) (width 0.75) (layer "F.Cu") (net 35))
 (segment (start 147.765 56.7) (end 147.775 56.69) (width 0.75) (layer "F.Cu") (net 35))
 (segment (start 147.765 54.16) (end 147.775 54.15) (width 0.75) (layer "F.Cu") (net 36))
 (segment (start 141.025 54.225) (end 143.453 54.225) (width 0.75) (layer "F.Cu") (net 36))
 (segment (start 143.453 54.225) (end 143.518 54.16) (width 0.75) (layer "F.Cu") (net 36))
 (segment (start 143.518 54.16) (end 147.765 54.16) (width 0.75) (layer "F.Cu") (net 36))
 (segment (start 143.772 51.62) (end 147.765 51.62) (width 0.75) (layer "F.Cu") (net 37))
 (segment (start 147.765 51.62) (end 147.775 51.61) (width 0.75) (layer "F.Cu") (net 37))
 (segment (start 147.765 49.08) (end 147.775 49.07) (width 0.75) (layer "F.Cu") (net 38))
 (segment (start 143.518 49.08) (end 147.765 49.08) (width 0.75) (layer "F.Cu") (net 38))
 (segment (start 147.765 46.54) (end 147.775 46.53) (width 0.75) (layer "F.Cu") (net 39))
 (segment (start 143.772 46.54) (end 147.765 46.54) (width 0.75) (layer "F.Cu") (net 39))
 (segment (start 143.518 44) (end 147.765 44) (width 0.75) (layer "F.Cu") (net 40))
 (segment (start 147.765 44) (end 147.775 43.99) (width 0.75) (layer "F.Cu") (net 40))
 (segment (start 128.532 44) (end 124.225 44) (width 0.75) (layer "F.Cu") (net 1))
 (segment (start 128.278 46.54) (end 124.225 46.54) (width 0.75) (layer "F.Cu") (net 2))
 (segment (start 128.532 49.08) (end 124.225 49.08) (width 0.75) (layer "F.Cu") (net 3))
 (segment (start 128.278 51.62) (end 124.225 51.62) (width 0.75) (layer "F.Cu") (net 4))
 (segment (start 128.532 54.16) (end 124.225 54.16) (width 0.75) (layer "F.Cu") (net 5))
 (segment (start 128.278 56.7) (end 124.225 56.7) (width 0.75) (layer "F.Cu") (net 6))
 (segment (start 128.532 59.24) (end 124.225 59.24) (width 0.75) (layer "F.Cu") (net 7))
 (segment (start 128.278 61.78) (end 124.225 61.78) (width 0.75) (layer "F.Cu") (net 8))
 (segment (start 128.532 64.32) (end 124.225 64.32) (width 0.75) (layer "F.Cu") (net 9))
 (segment (start 128.278 66.86) (end 124.225 66.86) (width 0.75) (layer "F.Cu") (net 10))
 (segment (start 128.532 69.4) (end 124.225 69.4) (width 0.75) (layer "F.Cu") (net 11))
 (segment (start 128.278 71.94) (end 124.225 71.94) (width 0.75) (layer "F.Cu") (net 12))
 (segment (start 128.532 74.48) (end 124.225 74.48) (width 0.75) (layer "F.Cu") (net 13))
 (segment (start 128.278 77.02) (end 124.225 77.02) (width 0.75) (layer "F.Cu") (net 14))
 (segment (start 128.532 79.56) (end 124.225 79.56) (width 0.75) (layer "F.Cu") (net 15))
 (segment (start 128.278 82.1) (end 124.225 82.1) (width 0.75) (layer "F.Cu") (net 16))
 (segment (start 128.532 84.64) (end 124.225 84.64) (width 0.75) (layer "F.Cu") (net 17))
 (segment (start 128.278 87.18) (end 124.225 87.18) (width 0.75) (layer "F.Cu") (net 18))
 (segment (start 128.532 89.72) (end 124.225 89.72) (width 0.75) (layer "F.Cu") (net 19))
 (segment (start 132.625 66.825) (end 132.625 68.525978) (width 0.75) (layer "F.Cu") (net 19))
 (segment (start 130.046311 71.104667) (end 130.046311 88.205689) (width 0.75) (layer "F.Cu") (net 19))
 (segment (start 130.046311 88.205689) (end 128.532 89.72) (width 0.75) (layer "F.Cu") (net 19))
 (segment (start 132.625 68.525978) (end 130.046311 71.104667) (width 0.75) (layer "F.Cu") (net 19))
 (segment (start 128.278 92.26) (end 124.225 92.26) (width 0.75) (layer "F.Cu") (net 20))
 (segment (start 139.725 43.525) (end 139.725 54.225) (width 0.75) (layer "F.Cu") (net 46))
 (segment (start 140.15 61.775) (end 140.175 61.8) (width 0.75) (layer "F.Cu") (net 46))
 (segment (start 138.45 61.775) (end 140.15 61.775) (width 0.75) (layer "F.Cu") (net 46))
 (segment (start 59.175 66.625) (end 59.2 66.6) (width 0.75) (layer "F.Cu") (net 46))
 (segment (start 59.2 48.09045) (end 68.46497 38.82548) (width 0.75) (layer "F.Cu") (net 46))
 (segment (start 139.7 54.225) (end 137.425 56.5) (width 0.75) (layer "F.Cu") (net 46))
 (segment (start 59.2 66.6) (end 59.2 48.09045) (width 0.75) (layer "F.Cu") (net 46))
 (segment (start 137.55 60.875) (end 138.45 61.775) (width 0.75) (layer "F.Cu") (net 46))
 (segment (start 68.46497 38.82548) (end 135.02548 38.82548) (width 0.75) (layer "F.Cu") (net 46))
 (segment (start 59.175 113.65) (end 59.175 66.625) (width 0.75) (layer "F.Cu") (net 46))
 (segment (start 139.725 54.225) (end 139.7 54.225) (width 0.75) (layer "F.Cu") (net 46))
 (segment (start 135.02548 38.82548) (end 139.725 43.525) (width 0.75) (layer "F.Cu") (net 46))
 (via (at 137.425 56.5) (size 0.8) (drill 0.4) (layers "F.Cu" "B.Cu") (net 46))
 (via (at 137.55 60.875) (size 0.8) (drill 0.4) (layers "F.Cu" "B.Cu") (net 46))
 (segment (start 137.425 56.5) (end 137.425 60.75) (width 0.75) (layer "B.Cu") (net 46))
 (segment (start 137.425 60.75) (end 137.55 60.875) (width 0.75) (layer "B.Cu") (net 46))
 (segment (start 69.2 41.6) (end 69.2 88.625) (width 0.75) (layer "F.Cu") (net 45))
 (segment (start 131.325 42.85) (end 128.525 40.05) (width 0.75) (layer "F.Cu") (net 45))
 (segment (start 69.2 88.625) (end 69.175 88.65) (width 0.75) (layer "F.Cu") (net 45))
 (segment (start 128.525 40.05) (end 70.75 40.05) (width 0.75) (layer "F.Cu") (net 45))
 (segment (start 131.325 64.825) (end 139.725 56.425) (width 0.75) (layer "F.Cu") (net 45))
 (segment (start 131.325 66.825) (end 131.325 64.825) (width 0.75) (layer "F.Cu") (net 45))
 (segment (start 131.325 64.825) (end 131.325 42.85) (width 0.75) (layer "F.Cu") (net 45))
 (segment (start 70.75 40.05) (end 69.2 41.6) (width 0.75) (layer "F.Cu") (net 45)))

